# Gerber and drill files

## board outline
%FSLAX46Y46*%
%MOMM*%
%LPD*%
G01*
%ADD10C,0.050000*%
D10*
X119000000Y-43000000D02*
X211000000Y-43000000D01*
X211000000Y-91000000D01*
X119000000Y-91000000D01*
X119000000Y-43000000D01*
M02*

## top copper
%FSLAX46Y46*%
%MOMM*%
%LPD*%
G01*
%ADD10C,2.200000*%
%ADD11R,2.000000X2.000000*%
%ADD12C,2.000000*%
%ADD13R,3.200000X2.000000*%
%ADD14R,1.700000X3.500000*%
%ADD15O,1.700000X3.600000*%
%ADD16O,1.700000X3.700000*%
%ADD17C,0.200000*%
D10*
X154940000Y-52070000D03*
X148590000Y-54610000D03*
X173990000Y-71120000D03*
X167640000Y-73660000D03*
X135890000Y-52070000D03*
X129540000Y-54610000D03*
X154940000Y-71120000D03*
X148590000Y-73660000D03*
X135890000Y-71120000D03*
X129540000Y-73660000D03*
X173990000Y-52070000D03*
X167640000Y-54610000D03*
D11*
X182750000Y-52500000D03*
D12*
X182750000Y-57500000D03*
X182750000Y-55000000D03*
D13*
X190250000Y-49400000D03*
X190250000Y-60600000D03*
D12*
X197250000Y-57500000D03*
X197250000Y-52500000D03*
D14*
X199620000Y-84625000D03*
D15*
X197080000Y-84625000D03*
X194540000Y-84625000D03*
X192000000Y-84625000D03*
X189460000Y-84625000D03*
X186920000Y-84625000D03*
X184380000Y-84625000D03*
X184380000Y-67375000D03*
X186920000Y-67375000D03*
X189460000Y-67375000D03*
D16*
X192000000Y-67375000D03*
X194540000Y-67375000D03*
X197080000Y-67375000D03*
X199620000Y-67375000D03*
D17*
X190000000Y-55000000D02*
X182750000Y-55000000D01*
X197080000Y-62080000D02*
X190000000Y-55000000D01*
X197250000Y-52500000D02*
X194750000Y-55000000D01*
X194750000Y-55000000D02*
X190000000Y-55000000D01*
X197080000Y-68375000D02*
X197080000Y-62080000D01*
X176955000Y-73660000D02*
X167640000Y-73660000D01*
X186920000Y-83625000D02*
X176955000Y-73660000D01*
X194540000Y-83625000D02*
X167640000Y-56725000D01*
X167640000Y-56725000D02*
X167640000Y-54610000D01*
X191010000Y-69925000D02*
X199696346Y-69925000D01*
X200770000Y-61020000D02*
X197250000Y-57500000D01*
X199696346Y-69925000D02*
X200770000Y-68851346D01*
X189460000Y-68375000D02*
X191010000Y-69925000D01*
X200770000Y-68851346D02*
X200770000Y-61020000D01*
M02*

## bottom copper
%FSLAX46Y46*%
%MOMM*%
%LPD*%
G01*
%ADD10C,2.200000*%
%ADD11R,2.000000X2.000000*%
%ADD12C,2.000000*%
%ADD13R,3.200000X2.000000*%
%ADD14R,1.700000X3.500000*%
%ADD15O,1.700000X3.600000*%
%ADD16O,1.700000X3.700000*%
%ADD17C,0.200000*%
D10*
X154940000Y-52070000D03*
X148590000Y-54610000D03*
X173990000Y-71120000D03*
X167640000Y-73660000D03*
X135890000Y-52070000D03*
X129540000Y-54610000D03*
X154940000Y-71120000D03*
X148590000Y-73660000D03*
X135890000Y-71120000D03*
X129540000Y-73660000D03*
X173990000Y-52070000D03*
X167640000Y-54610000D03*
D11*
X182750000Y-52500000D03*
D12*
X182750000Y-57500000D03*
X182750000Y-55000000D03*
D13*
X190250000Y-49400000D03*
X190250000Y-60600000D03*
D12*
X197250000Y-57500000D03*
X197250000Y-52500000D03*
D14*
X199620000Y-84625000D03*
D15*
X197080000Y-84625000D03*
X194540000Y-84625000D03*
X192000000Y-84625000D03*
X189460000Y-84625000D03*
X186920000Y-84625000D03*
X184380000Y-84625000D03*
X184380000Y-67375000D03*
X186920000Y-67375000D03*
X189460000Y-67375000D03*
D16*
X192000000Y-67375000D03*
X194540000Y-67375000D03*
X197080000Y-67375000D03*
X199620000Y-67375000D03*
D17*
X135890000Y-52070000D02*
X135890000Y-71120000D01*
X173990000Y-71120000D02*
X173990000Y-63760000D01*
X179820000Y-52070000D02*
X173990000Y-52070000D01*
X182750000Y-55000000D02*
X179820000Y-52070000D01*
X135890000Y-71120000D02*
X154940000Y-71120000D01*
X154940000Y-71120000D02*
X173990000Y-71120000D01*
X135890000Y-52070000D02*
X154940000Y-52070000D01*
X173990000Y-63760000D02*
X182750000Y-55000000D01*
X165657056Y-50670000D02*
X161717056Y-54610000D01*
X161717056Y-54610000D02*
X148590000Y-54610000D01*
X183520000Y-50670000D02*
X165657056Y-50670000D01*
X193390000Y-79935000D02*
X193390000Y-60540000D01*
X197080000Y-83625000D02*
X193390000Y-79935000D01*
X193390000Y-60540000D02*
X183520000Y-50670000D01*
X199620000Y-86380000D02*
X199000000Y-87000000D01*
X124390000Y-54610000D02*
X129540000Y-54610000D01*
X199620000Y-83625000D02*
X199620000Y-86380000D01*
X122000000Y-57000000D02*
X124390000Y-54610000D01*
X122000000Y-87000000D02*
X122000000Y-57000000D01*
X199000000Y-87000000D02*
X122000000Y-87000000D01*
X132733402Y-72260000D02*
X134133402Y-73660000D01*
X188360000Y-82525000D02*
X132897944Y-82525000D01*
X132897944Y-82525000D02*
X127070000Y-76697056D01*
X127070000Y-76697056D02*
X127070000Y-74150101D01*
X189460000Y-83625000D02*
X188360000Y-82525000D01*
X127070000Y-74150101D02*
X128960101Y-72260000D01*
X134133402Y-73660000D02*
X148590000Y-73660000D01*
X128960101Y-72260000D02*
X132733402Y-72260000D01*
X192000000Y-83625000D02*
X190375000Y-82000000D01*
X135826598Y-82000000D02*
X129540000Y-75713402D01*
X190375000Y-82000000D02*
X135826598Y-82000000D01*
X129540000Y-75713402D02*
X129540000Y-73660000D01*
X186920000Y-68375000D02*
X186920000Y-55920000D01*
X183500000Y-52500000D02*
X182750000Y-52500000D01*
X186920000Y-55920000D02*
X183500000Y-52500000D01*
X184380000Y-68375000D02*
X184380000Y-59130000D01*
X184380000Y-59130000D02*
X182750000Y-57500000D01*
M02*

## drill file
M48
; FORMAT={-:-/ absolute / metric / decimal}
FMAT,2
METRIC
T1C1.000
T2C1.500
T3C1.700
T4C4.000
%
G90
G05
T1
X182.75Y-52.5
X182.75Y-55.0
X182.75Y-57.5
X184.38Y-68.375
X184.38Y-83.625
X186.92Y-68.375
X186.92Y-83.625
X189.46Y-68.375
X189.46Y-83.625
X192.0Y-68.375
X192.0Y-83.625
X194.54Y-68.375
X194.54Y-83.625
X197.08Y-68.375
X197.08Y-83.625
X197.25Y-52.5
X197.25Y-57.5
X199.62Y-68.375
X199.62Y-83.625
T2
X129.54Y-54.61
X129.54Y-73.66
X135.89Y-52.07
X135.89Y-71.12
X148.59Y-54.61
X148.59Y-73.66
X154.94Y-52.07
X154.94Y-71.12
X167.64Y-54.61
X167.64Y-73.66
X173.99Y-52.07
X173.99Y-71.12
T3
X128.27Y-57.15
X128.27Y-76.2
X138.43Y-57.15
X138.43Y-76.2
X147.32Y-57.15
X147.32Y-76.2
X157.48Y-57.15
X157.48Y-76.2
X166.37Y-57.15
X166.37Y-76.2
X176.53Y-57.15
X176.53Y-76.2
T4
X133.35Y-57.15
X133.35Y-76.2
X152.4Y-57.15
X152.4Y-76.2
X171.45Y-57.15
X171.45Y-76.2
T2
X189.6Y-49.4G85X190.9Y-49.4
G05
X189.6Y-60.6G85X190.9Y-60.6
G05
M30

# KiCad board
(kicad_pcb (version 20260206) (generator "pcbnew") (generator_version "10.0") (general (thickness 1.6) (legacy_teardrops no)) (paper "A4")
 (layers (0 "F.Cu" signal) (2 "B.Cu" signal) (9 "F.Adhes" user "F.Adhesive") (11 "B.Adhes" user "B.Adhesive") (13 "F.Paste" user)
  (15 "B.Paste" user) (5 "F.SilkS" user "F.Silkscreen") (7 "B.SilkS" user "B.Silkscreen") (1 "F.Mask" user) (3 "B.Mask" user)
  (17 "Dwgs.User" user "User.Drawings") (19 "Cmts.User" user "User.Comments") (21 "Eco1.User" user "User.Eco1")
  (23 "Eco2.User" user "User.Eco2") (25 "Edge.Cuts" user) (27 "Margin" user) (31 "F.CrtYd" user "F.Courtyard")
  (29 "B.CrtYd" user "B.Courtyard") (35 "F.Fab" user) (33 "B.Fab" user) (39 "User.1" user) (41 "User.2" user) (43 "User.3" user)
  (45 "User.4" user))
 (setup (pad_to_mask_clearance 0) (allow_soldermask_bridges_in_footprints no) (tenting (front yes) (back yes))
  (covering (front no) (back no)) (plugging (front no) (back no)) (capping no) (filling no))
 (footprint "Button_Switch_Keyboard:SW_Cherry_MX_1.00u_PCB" (layer "F.Cu") (at 154.94 52.07)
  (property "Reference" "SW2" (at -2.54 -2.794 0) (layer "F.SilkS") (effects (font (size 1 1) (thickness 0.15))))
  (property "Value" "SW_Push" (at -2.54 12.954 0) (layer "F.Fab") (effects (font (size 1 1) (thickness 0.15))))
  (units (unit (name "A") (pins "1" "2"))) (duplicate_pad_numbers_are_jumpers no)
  (pad "" np_thru_hole circle (at -7.62 5.08) (size 1.7 1.7) (drill 1.7) (layers "*.Cu" "*.Mask"))
  (pad "" np_thru_hole circle (at -2.54 5.08) (size 4 4) (drill 4) (layers "*.Cu" "*.Mask"))
  (pad "" np_thru_hole circle (at 2.54 5.08) (size 1.7 1.7) (drill 1.7) (layers "*.Cu" "*.Mask"))
  (pad "1" thru_hole circle (at 0 0) (size 2.2 2.2) (drill 1.5) (layers "*.Cu" "*.Mask") (remove_unused_layers no) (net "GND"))
  (pad "2" thru_hole circle (at -6.35 2.54) (size 2.2 2.2) (drill 1.5) (layers "*.Cu" "*.Mask") (remove_unused_layers no)
   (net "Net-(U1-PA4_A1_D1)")))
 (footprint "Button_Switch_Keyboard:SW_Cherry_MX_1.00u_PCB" (layer "F.Cu") (at 173.99 71.12)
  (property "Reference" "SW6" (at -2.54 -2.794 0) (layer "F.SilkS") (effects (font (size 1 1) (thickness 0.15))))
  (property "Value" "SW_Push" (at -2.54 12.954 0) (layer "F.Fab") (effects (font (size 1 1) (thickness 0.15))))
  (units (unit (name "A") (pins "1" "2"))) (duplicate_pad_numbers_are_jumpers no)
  (pad "" np_thru_hole circle (at -7.62 5.08) (size 1.7 1.7) (drill 1.7) (layers "*.Cu" "*.Mask"))
  (pad "" np_thru_hole circle (at -2.54 5.08) (size 4 4) (drill 4) (layers "*.Cu" "*.Mask"))
  (pad "" np_thru_hole circle (at 2.54 5.08) (size 1.7 1.7) (drill 1.7) (layers "*.Cu" "*.Mask"))
  (pad "1" thru_hole circle (at 0 0) (size 2.2 2.2) (drill 1.5) (layers "*.Cu" "*.Mask") (remove_unused_layers no) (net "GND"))
  (pad "2" thru_hole circle (at -6.35 2.54) (size 2.2 2.2) (drill 1.5) (layers "*.Cu" "*.Mask") (remove_unused_layers no)
   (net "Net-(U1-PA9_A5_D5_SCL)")))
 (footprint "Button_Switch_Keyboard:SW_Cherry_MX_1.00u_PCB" (layer "F.Cu") (at 135.89 52.07)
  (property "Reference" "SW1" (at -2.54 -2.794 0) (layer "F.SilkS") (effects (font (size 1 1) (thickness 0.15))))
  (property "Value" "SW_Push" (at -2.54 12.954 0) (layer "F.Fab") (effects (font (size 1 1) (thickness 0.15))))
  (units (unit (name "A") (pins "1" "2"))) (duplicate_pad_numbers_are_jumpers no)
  (pad "" np_thru_hole circle (at -7.62 5.08) (size 1.7 1.7) (drill 1.7) (layers "*.Cu" "*.Mask"))
  (pad "" np_thru_hole circle (at -2.54 5.08) (size 4 4) (drill 4) (layers "*.Cu" "*.Mask"))
  (pad "" np_thru_hole circle (at 2.54 5.08) (size 1.7 1.7) (drill 1.7) (layers "*.Cu" "*.Mask"))
  (pad "1" thru_hole circle (at 0 0) (size 2.2 2.2) (drill 1.5) (layers "*.Cu" "*.Mask") (remove_unused_layers no) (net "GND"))
  (pad "2" thru_hole circle (at -6.35 2.54) (size 2.2 2.2) (drill 1.5) (layers "*.Cu" "*.Mask") (remove_unused_layers no)
   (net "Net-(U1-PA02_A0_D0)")))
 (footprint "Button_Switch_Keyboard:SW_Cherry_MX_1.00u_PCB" (layer "F.Cu") (at 154.94 71.12)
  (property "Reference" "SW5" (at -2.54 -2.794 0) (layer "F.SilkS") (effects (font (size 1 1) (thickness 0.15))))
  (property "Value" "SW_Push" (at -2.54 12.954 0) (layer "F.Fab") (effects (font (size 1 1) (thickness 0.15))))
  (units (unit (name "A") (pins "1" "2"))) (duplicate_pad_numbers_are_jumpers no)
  (pad "" np_thru_hole circle (at -7.62 5.08) (size 1.7 1.7) (drill 1.7) (layers "*.Cu" "*.Mask"))
  (pad "" np_thru_hole circle (at -2.54 5.08) (size 4 4) (drill 4) (layers "*.Cu" "*.Mask"))
  (pad "" np_thru_hole circle (at 2.54 5.08) (size 1.7 1.7) (drill 1.7) (layers "*.Cu" "*.Mask"))
  (pad "1" thru_hole circle (at 0 0) (size 2.2 2.2) (drill 1.5) (layers "*.Cu" "*.Mask") (remove_unused_layers no) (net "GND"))
  (pad "2" thru_hole circle (at -6.35 2.54) (size 2.2 2.2) (drill 1.5) (layers "*.Cu" "*.Mask") (remove_unused_layers no)
   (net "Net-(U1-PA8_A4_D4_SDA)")))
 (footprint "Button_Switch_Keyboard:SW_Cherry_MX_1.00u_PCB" (layer "F.Cu") (at 135.89 71.12)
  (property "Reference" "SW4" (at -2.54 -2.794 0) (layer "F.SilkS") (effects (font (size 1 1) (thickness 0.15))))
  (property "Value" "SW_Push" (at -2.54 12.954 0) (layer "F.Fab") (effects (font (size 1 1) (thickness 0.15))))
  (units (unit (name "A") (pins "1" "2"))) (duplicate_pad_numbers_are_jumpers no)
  (pad "" np_thru_hole circle (at -7.62 5.08) (size 1.7 1.7) (drill 1.7) (layers "*.Cu" "*.Mask"))
  (pad "" np_thru_hole circle (at -2.54 5.08) (size 4 4) (drill 4) (layers "*.Cu" "*.Mask"))
  (pad "" np_thru_hole circle (at 2.54 5.08) (size 1.7 1.7) (drill 1.7) (layers "*.Cu" "*.Mask"))
  (pad "1" thru_hole circle (at 0 0) (size 2.2 2.2) (drill 1.5) (layers "*.Cu" "*.Mask") (remove_unused_layers no) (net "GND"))
  (pad "2" thru_hole circle (at -6.35 2.54) (size 2.2 2.2) (drill 1.5) (layers "*.Cu" "*.Mask") (remove_unused_layers no)
   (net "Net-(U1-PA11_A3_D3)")))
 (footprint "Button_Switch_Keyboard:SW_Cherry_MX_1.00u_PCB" (layer "F.Cu") (at 173.99 52.07)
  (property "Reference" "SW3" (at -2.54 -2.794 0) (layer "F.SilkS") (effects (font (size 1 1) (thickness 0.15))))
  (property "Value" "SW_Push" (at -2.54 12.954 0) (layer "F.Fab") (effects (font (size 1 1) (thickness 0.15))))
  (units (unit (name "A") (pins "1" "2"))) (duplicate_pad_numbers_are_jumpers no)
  (pad "" np_thru_hole circle (at -7.62 5.08) (size 1.7 1.7) (drill 1.7) (layers "*.Cu" "*.Mask"))
  (pad "" np_thru_hole circle (at -2.54 5.08) (size 4 4) (drill 4) (layers "*.Cu" "*.Mask"))
  (pad "" np_thru_hole circle (at 2.54 5.08) (size 1.7 1.7) (drill 1.7) (layers "*.Cu" "*.Mask"))
  (pad "1" thru_hole circle (at 0 0) (size 2.2 2.2) (drill 1.5) (layers "*.Cu" "*.Mask") (remove_unused_layers no) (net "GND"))
  (pad "2" thru_hole circle (at -6.35 2.54) (size 2.2 2.2) (drill 1.5) (layers "*.Cu" "*.Mask") (remove_unused_layers no)
   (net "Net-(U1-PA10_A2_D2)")))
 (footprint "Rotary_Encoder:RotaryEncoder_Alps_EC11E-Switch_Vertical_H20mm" (layer "F.Cu") (at 182.75 52.5)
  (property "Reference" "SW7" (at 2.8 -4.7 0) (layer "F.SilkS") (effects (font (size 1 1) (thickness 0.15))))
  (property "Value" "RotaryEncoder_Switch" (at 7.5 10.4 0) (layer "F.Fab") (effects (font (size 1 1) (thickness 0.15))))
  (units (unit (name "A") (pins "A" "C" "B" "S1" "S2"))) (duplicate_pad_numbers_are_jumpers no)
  (pad "A" thru_hole rect (at 0 0) (size 2 2) (drill 1) (layers "*.Cu" "*.Mask") (remove_unused_layers no) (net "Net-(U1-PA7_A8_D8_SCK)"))
  (pad "B" thru_hole circle (at 0 5) (size 2 2) (drill 1) (layers "*.Cu" "*.Mask") (remove_unused_layers no) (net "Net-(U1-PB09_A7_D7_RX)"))
  (pad "C" thru_hole circle (at 0 2.5) (size 2 2) (drill 1) (layers "*.Cu" "*.Mask") (remove_unused_layers no) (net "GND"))
  (pad "MP" thru_hole rect (at 7.5 -3.1) (size 3.2 2) (drill oval 2.8 1.5) (layers "*.Cu" "*.Mask") (remove_unused_layers no))
  (pad "MP" thru_hole rect (at 7.5 8.1) (size 3.2 2) (drill oval 2.8 1.5) (layers "*.Cu" "*.Mask") (remove_unused_layers no))
  (pad "S1" thru_hole circle (at 14.5 5) (size 2 2) (drill 1) (layers "*.Cu" "*.Mask") (remove_unused_layers no)
   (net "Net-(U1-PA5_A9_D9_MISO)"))
  (pad "S2" thru_hole circle (at 14.5 0) (size 2 2) (drill 1) (layers "*.Cu" "*.Mask") (remove_unused_layers no) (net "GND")))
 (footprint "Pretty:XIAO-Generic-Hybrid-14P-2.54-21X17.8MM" (layer "B.Cu") (at 192 76 90)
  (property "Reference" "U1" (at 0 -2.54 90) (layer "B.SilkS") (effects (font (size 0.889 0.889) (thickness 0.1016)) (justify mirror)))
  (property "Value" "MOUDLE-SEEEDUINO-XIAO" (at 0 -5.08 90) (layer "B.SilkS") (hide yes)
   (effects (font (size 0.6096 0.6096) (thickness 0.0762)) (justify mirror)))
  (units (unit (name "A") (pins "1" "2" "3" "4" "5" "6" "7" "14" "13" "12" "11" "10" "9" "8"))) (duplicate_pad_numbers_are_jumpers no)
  (pad "1" thru_hole rect (at -7.625 7.62 90) (size 3.5 1.7) (drill 1 (offset -1 0)) (layers "*.Cu" "*.Mask") (remove_unused_layers no)
   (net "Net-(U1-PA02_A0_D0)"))
  (pad "2" thru_hole oval (at -7.625 5.08 90) (size 3.6 1.7) (drill 1 (offset -1 0)) (layers "*.Cu" "*.Mask") (remove_unused_layers no)
   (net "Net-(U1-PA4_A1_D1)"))
  (pad "3" thru_hole oval (at -7.625 2.54 90) (size 3.6 1.7) (drill 1 (offset -1 0)) (layers "*.Cu" "*.Mask") (remove_unused_layers no)
   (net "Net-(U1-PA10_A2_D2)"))
  (pad "4" thru_hole oval (at -7.625 0 90) (size 3.6 1.7) (drill 1 (offset -1 0)) (layers "*.Cu" "*.Mask") (remove_unused_layers no)
   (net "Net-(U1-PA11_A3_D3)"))
  (pad "5" thru_hole oval (at -7.625 -2.54 90) (size 3.6 1.7) (drill 1 (offset -1 0)) (layers "*.Cu" "*.Mask") (remove_unused_layers no)
   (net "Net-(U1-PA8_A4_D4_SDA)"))
  (pad "6" thru_hole oval (at -7.625 -5.08 270) (size 3.6 1.7) (drill 1 (offset 1 0)) (layers "*.Cu" "*.Mask") (remove_unused_layers no)
   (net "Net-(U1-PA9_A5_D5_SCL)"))
  (pad "7" thru_hole oval (at -7.625 -7.62 90) (size 3.6 1.7) (drill 1 (offset -1 0)) (layers "*.Cu" "*.Mask") (remove_unused_layers no)
   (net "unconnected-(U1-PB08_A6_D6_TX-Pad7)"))
  (pad "8" thru_hole oval (at 7.625 -7.62 90) (size 3.6 1.7) (drill 1 (offset 1 0)) (layers "*.Cu" "*.Mask") (remove_unused_layers no)
   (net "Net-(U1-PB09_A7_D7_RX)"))
  (pad "9" thru_hole oval (at 7.625 -5.08 90) (size 3.6 1.7) (drill 1 (offset 1 0)) (layers "*.Cu" "*.Mask") (remove_unused_layers no)
   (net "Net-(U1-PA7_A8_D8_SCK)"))
  (pad "10" thru_hole oval (at 7.625 -2.54 90) (size 3.6 1.7) (drill 1 (offset 1 0)) (layers "*.Cu" "*.Mask") (remove_unused_layers no)
   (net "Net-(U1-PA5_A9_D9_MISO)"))
  (pad "11" thru_hole oval (at 7.625 0 90) (size 3.7 1.7) (drill 1 (offset 1 0)) (layers "*.Cu" "*.Mask") (remove_unused_layers no)
   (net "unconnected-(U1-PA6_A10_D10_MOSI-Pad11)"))
  (pad "12" thru_hole oval (at 7.625 2.54 90) (size 3.7 1.7) (drill 1 (offset 1 0)) (layers "*.Cu" "*.Mask") (remove_unused_layers no)
   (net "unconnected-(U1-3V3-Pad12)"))
  (pad "13" thru_hole oval (at 7.625 5.08 90) (size 3.7 1.7) (drill 1 (offset 1 0)) (layers "*.Cu" "*.Mask") (remove_unused_layers no)
   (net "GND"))
  (pad "14" thru_hole oval (at 7.625 7.62 90) (size 3.7 1.7) (drill 1 (offset 1 0)) (layers "*.Cu" "*.Mask") (remove_unused_layers no)
   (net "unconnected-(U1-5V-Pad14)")))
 (gr_rect (start 119 43) (end 211 91) (stroke (width 0.05) (type default)) (fill no) (layer "Edge.Cuts"))
 (segment (start 190 55) (end 182.75 55) (width 0.2) (layer "F.Cu") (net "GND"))
 (segment (start 197.08 62.08) (end 190 55) (width 0.2) (layer "F.Cu") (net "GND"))
 (segment (start 197.25 52.5) (end 194.75 55) (width 0.2) (layer "F.Cu") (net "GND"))
 (segment (start 194.75 55) (end 190 55) (width 0.2) (layer "F.Cu") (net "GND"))
 (segment (start 197.08 68.375) (end 197.08 62.08) (width 0.2) (layer "F.Cu") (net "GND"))
 (segment (start 135.89 52.07) (end 135.89 71.12) (width 0.2) (layer "B.Cu") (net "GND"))
 (segment (start 173.99 71.12) (end 173.99 63.76) (width 0.2) (layer "B.Cu") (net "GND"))
 (segment (start 179.82 52.07) (end 173.99 52.07) (width 0.2) (layer "B.Cu") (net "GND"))
 (segment (start 182.75 55) (end 179.82 52.07) (width 0.2) (layer "B.Cu") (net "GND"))
 (segment (start 135.89 71.12) (end 154.94 71.12) (width 0.2) (layer "B.Cu") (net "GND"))
 (segment (start 154.94 71.12) (end 173.99 71.12) (width 0.2) (layer "B.Cu") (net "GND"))
 (segment (start 135.89 52.07) (end 154.94 52.07) (width 0.2) (layer "B.Cu") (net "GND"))
 (segment (start 173.99 63.76) (end 182.75 55) (width 0.2) (layer "B.Cu") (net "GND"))
 (segment (start 165.657056 50.67) (end 161.717056 54.61) (width 0.2) (layer "B.Cu") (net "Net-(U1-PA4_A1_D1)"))
 (segment (start 161.717056 54.61) (end 148.59 54.61) (width 0.2) (layer "B.Cu") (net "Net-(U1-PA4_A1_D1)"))
 (segment (start 183.52 50.67) (end 165.657056 50.67) (width 0.2) (layer "B.Cu") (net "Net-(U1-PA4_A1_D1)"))
 (segment (start 193.39 79.935) (end 193.39 60.54) (width 0.2) (layer "B.Cu") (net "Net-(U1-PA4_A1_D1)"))
 (segment (start 197.08 83.625) (end 193.39 79.935) (width 0.2) (layer "B.Cu") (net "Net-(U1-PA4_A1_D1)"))
 (segment (start 193.39 60.54) (end 183.52 50.67) (width 0.2) (layer "B.Cu") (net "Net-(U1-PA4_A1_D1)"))
 (segment (start 176.955 73.66) (end 167.64 73.66) (width 0.2) (layer "F.Cu") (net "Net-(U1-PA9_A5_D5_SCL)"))
 (segment (start 186.92 83.625) (end 176.955 73.66) (width 0.2) (layer "F.Cu") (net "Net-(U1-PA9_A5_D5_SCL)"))
 (segment (start 199.62 86.38) (end 199 87) (width 0.2) (layer "B.Cu") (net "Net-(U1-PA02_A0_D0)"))
 (segment (start 124.39 54.61) (end 129.54 54.61) (width 0.2) (layer "B.Cu") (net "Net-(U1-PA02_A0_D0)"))
 (segment (start 199.62 83.625) (end 199.62 86.38) (width 0.2) (layer "B.Cu") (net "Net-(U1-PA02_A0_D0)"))
 (segment (start 122 57) (end 124.39 54.61) (width 0.2) (layer "B.Cu") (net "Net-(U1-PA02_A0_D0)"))
 (segment (start 122 87) (end 122 57) (width 0.2) (layer "B.Cu") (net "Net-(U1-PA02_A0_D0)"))
 (segment (start 199 87) (end 122 87) (width 0.2) (layer "B.Cu") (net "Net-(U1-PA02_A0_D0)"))
 (segment (start 132.733402 72.26) (end 134.133402 73.66) (width 0.2) (layer "B.Cu") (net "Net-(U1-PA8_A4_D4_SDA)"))
 (segment (start 188.36 82.525) (end 132.897944 82.525) (width 0.2) (layer "B.Cu") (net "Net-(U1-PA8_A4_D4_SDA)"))
 (segment (start 132.897944 82.525) (end 127.07 76.697056) (width 0.2) (layer "B.Cu") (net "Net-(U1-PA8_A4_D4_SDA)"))
 (segment (start 127.07 76.697056) (end 127.07 74.150101) (width 0.2) (layer "B.Cu") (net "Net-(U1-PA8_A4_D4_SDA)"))
 (segment (start 189.46 83.625) (end 188.36 82.525) (width 0.2) (layer "B.Cu") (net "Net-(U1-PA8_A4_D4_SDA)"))
 (segment (start 127.07 74.150101) (end 128.960101 72.26) (width 0.2) (layer "B.Cu") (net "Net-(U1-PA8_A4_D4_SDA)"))
 (segment (start 134.133402 73.66) (end 148.59 73.66) (width 0.2) (layer "B.Cu") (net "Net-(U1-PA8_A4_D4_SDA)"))
 (segment (start 128.960101 72.26) (end 132.733402 72.26) (width 0.2) (layer "B.Cu") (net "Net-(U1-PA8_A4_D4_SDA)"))
 (segment (start 192 83.625) (end 190.375 82) (width 0.2) (layer "B.Cu") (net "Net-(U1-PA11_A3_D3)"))
 (segment (start 135.826598 82) (end 129.54 75.713402) (width 0.2) (layer "B.Cu") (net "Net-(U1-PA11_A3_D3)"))
 (segment (start 190.375 82) (end 135.826598 82) (width 0.2) (layer "B.Cu") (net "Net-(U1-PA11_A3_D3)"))
 (segment (start 129.54 75.713402) (end 129.54 73.66) (width 0.2) (layer "B.Cu") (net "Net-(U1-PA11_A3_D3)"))
 (segment (start 194.54 83.625) (end 167.64 56.725) (width 0.2) (layer "F.Cu") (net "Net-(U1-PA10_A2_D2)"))
 (segment (start 167.64 56.725) (end 167.64 54.61) (width 0.2) (layer "F.Cu") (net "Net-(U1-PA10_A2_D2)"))
 (segment (start 186.92 68.375) (end 186.92 55.92) (width 0.2) (layer "B.Cu") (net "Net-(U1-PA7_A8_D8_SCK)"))
 (segment (start 183.5 52.5) (end 182.75 52.5) (width 0.2) (layer "B.Cu") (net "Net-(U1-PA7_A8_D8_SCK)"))
 (segment (start 186.92 55.92) (end 183.5 52.5) (width 0.2) (layer "B.Cu") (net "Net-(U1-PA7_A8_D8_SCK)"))
 (segment (start 184.38 68.375) (end 184.38 59.13) (width 0.2) (layer "B.Cu") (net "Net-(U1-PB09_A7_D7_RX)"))
 (segment (start 184.38 59.13) (end 182.75 57.5) (width 0.2) (layer "B.Cu") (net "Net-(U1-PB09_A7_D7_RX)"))
 (segment (start 191.01 69.925) (end 199.696346 69.925) (width 0.2) (layer "F.Cu") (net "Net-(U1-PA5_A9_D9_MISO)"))
 (segment (start 200.77 61.02) (end 197.25 57.5) (width 0.2) (layer "F.Cu") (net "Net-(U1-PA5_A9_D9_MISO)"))
 (segment (start 199.696346 69.925) (end 200.77 68.851346) (width 0.2) (layer "F.Cu") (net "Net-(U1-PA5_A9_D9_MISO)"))
 (segment (start 189.46 68.375) (end 191.01 69.925) (width 0.2) (layer "F.Cu") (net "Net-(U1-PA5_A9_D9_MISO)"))
 (segment (start 200.77 68.851346) (end 200.77 61.02) (width 0.2) (layer "F.Cu") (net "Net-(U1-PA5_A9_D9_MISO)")))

